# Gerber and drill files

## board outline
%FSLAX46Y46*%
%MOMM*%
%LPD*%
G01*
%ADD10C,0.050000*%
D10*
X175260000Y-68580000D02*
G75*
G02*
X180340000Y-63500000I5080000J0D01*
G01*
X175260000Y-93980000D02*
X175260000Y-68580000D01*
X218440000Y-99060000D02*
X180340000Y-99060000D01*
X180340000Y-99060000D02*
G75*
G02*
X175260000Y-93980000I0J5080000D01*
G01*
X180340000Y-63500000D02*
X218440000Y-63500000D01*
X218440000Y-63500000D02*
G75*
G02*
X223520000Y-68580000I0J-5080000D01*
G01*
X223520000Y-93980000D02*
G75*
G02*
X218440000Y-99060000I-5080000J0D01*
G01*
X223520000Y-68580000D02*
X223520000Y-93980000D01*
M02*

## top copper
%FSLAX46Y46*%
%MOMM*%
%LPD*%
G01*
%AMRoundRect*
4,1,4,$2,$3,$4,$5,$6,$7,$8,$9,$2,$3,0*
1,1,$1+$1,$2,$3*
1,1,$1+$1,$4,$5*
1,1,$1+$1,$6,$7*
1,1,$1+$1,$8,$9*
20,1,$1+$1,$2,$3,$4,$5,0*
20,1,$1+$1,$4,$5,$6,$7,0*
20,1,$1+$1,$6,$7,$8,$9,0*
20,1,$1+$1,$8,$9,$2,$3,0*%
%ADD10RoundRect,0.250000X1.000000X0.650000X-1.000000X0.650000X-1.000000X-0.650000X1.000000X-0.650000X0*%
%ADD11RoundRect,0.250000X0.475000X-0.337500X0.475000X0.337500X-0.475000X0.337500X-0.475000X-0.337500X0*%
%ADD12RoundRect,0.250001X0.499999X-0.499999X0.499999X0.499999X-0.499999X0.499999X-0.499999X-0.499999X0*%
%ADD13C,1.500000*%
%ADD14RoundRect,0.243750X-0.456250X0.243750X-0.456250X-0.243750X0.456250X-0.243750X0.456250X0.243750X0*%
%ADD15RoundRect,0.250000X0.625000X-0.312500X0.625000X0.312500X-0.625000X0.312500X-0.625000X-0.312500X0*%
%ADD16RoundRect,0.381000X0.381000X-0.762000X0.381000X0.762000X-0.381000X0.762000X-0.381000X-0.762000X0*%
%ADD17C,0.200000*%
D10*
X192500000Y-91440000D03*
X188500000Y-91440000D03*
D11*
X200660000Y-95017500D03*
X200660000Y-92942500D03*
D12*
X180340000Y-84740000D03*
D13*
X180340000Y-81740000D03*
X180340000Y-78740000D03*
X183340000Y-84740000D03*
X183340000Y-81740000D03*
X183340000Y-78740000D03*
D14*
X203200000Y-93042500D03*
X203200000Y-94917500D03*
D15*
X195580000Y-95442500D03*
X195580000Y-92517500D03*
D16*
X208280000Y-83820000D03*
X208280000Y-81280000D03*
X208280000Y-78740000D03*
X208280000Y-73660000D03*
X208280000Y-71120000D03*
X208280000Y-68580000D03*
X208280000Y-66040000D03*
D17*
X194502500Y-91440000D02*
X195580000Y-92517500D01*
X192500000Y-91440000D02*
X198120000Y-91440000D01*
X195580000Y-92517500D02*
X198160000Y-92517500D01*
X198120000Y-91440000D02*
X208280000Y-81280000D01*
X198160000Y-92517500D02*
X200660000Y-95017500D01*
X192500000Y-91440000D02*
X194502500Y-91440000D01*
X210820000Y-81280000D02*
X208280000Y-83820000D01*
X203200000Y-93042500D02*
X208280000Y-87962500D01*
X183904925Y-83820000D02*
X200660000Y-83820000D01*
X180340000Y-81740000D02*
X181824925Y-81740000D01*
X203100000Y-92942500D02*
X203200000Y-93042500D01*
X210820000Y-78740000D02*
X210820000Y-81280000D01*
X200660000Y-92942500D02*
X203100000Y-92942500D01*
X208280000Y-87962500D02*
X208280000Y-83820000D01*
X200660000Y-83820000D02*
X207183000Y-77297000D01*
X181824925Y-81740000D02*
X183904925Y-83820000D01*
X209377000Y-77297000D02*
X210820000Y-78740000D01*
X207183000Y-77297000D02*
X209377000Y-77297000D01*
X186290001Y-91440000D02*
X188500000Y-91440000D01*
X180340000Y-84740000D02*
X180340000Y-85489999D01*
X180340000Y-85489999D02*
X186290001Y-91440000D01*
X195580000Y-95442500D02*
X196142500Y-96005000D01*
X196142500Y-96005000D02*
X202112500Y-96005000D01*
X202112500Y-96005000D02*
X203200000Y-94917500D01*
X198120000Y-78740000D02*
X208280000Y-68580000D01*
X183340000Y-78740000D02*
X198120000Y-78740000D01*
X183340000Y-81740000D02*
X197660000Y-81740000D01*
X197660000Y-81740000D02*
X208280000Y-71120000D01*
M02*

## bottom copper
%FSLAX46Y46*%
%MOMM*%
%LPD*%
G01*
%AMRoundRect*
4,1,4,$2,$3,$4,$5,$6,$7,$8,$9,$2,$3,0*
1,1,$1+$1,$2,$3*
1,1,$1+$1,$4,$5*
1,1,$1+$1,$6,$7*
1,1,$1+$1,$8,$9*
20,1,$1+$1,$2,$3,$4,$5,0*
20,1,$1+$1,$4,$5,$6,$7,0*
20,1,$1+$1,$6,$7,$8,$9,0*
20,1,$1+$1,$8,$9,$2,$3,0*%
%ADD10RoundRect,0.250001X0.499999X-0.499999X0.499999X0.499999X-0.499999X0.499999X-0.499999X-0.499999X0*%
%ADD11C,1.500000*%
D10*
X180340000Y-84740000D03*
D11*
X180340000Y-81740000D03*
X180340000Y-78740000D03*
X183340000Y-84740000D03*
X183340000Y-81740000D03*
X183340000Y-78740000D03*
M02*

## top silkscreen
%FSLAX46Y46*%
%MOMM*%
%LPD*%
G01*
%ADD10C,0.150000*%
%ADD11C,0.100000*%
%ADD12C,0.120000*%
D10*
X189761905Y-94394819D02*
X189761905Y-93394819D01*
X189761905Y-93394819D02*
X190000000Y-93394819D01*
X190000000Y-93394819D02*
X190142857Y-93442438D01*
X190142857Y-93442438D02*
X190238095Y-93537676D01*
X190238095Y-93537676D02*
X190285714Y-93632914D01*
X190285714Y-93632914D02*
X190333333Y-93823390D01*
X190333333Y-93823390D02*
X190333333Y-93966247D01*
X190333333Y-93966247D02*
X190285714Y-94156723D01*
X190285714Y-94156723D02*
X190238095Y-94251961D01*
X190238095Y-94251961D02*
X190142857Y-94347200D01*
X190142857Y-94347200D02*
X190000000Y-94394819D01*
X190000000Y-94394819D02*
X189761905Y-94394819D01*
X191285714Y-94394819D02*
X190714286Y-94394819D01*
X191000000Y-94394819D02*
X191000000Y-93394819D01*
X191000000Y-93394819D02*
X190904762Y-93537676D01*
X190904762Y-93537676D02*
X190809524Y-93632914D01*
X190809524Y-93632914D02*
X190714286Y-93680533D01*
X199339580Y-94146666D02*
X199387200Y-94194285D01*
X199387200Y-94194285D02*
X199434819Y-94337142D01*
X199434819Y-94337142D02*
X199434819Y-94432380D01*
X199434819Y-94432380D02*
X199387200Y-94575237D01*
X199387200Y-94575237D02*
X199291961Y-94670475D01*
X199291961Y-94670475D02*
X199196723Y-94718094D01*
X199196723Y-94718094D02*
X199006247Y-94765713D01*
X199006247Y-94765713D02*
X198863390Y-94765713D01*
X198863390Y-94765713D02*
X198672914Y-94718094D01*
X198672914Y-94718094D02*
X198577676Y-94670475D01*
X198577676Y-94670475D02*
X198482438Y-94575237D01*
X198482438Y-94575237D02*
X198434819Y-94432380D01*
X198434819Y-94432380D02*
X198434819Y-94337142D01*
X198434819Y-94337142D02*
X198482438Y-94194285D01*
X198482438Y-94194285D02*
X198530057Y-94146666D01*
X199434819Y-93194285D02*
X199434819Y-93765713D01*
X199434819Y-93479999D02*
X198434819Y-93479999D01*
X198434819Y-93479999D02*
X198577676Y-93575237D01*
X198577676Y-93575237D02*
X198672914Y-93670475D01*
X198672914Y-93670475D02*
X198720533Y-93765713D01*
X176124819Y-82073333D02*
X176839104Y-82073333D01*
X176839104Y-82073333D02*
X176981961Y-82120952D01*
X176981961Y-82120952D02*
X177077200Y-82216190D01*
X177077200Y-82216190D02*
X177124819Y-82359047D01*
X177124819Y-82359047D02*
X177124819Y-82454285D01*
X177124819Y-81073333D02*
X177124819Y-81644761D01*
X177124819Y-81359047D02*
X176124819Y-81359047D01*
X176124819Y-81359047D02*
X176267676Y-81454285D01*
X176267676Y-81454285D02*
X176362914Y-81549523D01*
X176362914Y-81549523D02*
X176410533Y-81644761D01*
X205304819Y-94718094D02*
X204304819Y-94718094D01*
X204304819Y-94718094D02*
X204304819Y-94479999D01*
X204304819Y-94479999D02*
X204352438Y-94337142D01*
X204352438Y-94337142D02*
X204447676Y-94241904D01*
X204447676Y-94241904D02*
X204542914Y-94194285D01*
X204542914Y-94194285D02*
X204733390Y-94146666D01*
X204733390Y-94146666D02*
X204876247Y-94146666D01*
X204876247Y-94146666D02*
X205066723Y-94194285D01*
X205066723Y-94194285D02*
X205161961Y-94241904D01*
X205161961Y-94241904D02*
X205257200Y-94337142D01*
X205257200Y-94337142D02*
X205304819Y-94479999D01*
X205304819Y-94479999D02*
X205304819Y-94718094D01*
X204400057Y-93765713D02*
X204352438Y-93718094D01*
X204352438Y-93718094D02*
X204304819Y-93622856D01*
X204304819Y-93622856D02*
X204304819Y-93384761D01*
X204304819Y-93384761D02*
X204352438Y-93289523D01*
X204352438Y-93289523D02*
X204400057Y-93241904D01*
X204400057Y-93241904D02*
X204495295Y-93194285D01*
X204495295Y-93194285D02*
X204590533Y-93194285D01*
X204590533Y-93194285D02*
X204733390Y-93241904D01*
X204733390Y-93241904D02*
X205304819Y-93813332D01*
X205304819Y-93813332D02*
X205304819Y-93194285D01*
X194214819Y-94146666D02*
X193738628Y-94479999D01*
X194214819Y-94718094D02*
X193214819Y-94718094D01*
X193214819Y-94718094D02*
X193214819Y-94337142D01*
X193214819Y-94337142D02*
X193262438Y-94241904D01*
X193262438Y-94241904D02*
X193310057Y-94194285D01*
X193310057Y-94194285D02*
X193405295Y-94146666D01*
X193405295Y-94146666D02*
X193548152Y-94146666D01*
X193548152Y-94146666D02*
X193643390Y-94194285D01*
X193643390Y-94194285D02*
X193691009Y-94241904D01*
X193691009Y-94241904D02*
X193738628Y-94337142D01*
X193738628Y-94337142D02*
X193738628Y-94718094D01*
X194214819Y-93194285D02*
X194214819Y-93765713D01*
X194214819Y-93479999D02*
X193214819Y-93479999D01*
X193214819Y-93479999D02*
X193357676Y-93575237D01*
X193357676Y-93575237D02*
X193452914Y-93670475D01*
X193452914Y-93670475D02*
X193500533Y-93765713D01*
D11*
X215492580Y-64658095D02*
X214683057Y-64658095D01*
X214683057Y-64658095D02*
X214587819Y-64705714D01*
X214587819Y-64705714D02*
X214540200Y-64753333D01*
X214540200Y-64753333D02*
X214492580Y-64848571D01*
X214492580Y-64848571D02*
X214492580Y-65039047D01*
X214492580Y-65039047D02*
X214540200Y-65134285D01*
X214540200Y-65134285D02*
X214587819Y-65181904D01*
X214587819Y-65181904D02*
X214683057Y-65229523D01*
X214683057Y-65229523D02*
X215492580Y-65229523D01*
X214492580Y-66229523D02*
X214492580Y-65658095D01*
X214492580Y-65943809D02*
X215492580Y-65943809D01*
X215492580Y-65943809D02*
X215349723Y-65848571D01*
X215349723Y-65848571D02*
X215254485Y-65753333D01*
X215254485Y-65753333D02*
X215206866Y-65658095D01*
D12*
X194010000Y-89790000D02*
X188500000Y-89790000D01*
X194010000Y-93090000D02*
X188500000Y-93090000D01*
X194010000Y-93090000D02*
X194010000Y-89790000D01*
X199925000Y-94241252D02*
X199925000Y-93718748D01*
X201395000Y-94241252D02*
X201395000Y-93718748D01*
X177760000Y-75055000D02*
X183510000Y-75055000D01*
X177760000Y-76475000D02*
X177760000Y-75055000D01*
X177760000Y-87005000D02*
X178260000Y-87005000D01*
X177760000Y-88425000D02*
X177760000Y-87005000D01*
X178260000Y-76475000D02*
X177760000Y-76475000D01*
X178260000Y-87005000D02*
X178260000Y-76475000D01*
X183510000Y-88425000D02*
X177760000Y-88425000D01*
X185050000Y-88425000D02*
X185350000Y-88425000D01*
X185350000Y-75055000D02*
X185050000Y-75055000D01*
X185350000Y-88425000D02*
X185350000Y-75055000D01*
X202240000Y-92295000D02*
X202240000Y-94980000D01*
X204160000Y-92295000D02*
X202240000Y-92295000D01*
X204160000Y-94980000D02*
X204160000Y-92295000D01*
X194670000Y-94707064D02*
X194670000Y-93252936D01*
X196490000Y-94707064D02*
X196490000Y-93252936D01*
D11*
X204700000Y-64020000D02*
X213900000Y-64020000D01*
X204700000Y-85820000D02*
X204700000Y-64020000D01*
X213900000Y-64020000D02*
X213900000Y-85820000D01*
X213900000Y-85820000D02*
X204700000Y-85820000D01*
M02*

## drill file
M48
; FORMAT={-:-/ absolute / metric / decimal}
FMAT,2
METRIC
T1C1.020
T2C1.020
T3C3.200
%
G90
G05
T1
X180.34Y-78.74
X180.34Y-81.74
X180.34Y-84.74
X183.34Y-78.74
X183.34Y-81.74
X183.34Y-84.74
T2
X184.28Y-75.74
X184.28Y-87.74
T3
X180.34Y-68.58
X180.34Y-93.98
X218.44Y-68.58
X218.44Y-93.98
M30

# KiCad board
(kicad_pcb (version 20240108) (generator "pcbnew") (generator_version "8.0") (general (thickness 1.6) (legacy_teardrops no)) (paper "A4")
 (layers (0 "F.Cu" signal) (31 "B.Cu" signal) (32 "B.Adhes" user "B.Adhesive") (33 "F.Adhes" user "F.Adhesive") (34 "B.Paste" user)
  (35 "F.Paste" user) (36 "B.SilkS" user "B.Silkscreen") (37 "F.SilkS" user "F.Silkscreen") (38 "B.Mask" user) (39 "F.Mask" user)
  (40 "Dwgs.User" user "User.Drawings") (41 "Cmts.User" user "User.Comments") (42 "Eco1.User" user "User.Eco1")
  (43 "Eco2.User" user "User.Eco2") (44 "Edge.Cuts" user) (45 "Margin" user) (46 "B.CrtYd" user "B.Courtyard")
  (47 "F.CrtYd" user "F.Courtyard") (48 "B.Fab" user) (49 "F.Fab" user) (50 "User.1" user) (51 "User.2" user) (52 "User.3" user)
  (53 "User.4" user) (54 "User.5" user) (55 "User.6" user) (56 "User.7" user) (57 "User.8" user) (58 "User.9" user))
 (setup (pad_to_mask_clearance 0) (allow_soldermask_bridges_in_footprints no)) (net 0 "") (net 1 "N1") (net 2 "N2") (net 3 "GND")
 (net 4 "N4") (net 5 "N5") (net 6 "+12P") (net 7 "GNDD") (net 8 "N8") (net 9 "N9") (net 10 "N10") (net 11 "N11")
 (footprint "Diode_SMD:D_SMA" (layer "F.Cu") (at 190.5 91.44 180)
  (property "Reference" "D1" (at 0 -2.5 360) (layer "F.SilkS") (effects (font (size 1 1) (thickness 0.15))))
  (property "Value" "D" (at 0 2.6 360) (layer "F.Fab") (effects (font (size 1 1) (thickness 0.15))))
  (fp_line (start -3.51 1.65) (end 2 1.65) (stroke (width 0.12) (type solid)) (layer "F.SilkS"))
  (fp_line (start -3.51 -1.65) (end 2 -1.65) (stroke (width 0.12) (type solid)) (layer "F.SilkS"))
  (fp_line (start -3.51 -1.65) (end -3.51 1.65) (stroke (width 0.12) (type solid)) (layer "F.SilkS"))
  (pad "1" smd roundrect (at -2 0 180) (size 2.5 1.8) (layers "F.Cu" "F.Paste" "F.Mask") (roundrect_rratio 0.1388888889) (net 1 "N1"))
  (pad "2" smd roundrect (at 2 0 180) (size 2.5 1.8) (layers "F.Cu" "F.Paste" "F.Mask") (roundrect_rratio 0.1388888889) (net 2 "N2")))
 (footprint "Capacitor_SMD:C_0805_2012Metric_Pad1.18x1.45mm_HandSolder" (layer "F.Cu") (at 200.66 93.98 90)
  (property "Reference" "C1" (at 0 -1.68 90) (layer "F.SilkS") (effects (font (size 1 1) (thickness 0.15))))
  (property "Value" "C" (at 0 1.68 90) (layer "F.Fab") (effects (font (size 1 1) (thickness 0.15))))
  (fp_line (start -0.261252 -0.735) (end 0.261252 -0.735) (stroke (width 0.12) (type solid)) (layer "F.SilkS"))
  (fp_line (start -0.261252 0.735) (end 0.261252 0.735) (stroke (width 0.12) (type solid)) (layer "F.SilkS"))
  (pad "1" smd roundrect (at -1.0375 0 90) (size 1.175 1.45) (layers "F.Cu" "F.Paste" "F.Mask") (roundrect_rratio 0.212766) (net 1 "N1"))
  (pad "2" smd roundrect (at 1.0375 0 90) (size 1.175 1.45) (layers "F.Cu" "F.Paste" "F.Mask") (roundrect_rratio 0.212766) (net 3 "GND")))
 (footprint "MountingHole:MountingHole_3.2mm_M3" (layer "F.Cu") (at 218.44 93.98)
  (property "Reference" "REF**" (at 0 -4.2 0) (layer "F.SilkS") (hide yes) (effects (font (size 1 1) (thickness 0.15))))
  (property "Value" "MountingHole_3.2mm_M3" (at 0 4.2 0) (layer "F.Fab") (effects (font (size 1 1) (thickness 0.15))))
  (pad "" np_thru_hole circle (at 0 0) (size 3.2 3.2) (drill 3.2) (layers "*.Cu" "*.Mask")))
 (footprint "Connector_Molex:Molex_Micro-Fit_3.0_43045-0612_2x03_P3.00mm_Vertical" (layer "F.Cu") (at 180.34 84.74 90)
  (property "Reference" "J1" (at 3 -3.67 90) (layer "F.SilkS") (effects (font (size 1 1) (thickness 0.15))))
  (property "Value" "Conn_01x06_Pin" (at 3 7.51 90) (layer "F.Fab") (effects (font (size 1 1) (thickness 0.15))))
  (fp_line (start 9.685 -2.58) (end 9.685 3.17) (stroke (width 0.12) (type solid)) (layer "F.SilkS"))
  (fp_line (start 8.265 -2.58) (end 9.685 -2.58) (stroke (width 0.12) (type solid)) (layer "F.SilkS"))
  (fp_line (start -2.265 -2.58) (end -2.265 -2.08) (stroke (width 0.12) (type solid)) (layer "F.SilkS"))
  (fp_line (start -3.685 -2.58) (end -2.265 -2.58) (stroke (width 0.12) (type solid)) (layer "F.SilkS"))
  (fp_line (start 8.265 -2.08) (end 8.265 -2.58) (stroke (width 0.12) (type solid)) (layer "F.SilkS"))
  (fp_line (start -2.265 -2.08) (end 8.265 -2.08) (stroke (width 0.12) (type solid)) (layer "F.SilkS"))
  (fp_line (start -3.685 3.17) (end -3.685 -2.58) (stroke (width 0.12) (type solid)) (layer "F.SilkS"))
  (fp_line (start -3.685 4.71) (end -3.685 5.01) (stroke (width 0.12) (type solid)) (layer "F.SilkS"))
  (fp_line (start 9.685 5.01) (end 9.685 4.71) (stroke (width 0.12) (type solid)) (layer "F.SilkS"))
  (fp_line (start -3.685 5.01) (end 9.685 5.01) (stroke (width 0.12) (type solid)) (layer "F.SilkS"))
  (pad "" np_thru_hole circle (at -3 3.94 90) (size 1.02 1.02) (drill 1.02) (layers "*.Cu" "*.Mask"))
  (pad "" np_thru_hole circle (at 9 3.94 90) (size 1.02 1.02) (drill 1.02) (layers "*.Cu" "*.Mask"))
  (pad "1" thru_hole roundrect (at 0 0 90) (size 1.5 1.5) (drill 1.02) (layers "*.Cu" "*.Mask") (remove_unused_layers no)
   (roundrect_rratio 0.166667) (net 2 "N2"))
  (pad "2" thru_hole circle (at 3 0 90) (size 1.5 1.5) (drill 1.02) (layers "*.Cu" "*.Mask") (remove_unused_layers no) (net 3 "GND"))
  (pad "3" thru_hole circle (at 6 0 90) (size 1.5 1.5) (drill 1.02) (layers "*.Cu" "*.Mask") (remove_unused_layers no) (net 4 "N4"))
  (pad "4" thru_hole circle (at 0 3 90) (size 1.5 1.5) (drill 1.02) (layers "*.Cu" "*.Mask") (remove_unused_layers no) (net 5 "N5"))
  (pad "5" thru_hole circle (at 3 3 90) (size 1.5 1.5) (drill 1.02) (layers "*.Cu" "*.Mask") (remove_unused_layers no) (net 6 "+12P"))
  (pad "6" thru_hole circle (at 6 3 90) (size 1.5 1.5) (drill 1.02) (layers "*.Cu" "*.Mask") (remove_unused_layers no) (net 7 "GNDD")))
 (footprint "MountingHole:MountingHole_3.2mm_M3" (layer "F.Cu") (at 180.34 93.98)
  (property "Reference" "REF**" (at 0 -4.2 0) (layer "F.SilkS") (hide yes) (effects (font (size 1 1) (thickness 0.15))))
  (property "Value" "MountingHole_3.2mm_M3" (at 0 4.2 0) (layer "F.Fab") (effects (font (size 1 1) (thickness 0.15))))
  (pad "" np_thru_hole circle (at 0 0) (size 3.2 3.2) (drill 3.2) (layers "*.Cu" "*.Mask")))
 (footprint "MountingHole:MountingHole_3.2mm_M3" (layer "F.Cu") (at 180.34 68.58)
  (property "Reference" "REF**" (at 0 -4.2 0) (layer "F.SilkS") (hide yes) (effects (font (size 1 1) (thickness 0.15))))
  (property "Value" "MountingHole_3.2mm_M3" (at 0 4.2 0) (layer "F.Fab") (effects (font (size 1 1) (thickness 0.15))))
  (pad "" np_thru_hole circle (at 0 0) (size 3.2 3.2) (drill 3.2) (layers "*.Cu" "*.Mask")))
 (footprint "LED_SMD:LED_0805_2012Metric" (layer "F.Cu") (at 203.2 93.98 -90)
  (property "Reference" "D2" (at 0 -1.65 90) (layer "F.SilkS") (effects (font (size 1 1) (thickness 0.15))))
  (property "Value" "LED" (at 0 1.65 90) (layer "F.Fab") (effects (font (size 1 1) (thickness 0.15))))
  (fp_line (start -1.685 0.96) (end 1 0.96) (stroke (width 0.12) (type solid)) (layer "F.SilkS"))
  (fp_line (start -1.685 -0.96) (end -1.685 0.96) (stroke (width 0.12) (type solid)) (layer "F.SilkS"))
  (fp_line (start 1 -0.96) (end -1.685 -0.96) (stroke (width 0.12) (type solid)) (layer "F.SilkS"))
  (pad "1" smd roundrect (at -0.9375 0 270) (size 0.975 1.4) (layers "F.Cu" "F.Paste" "F.Mask") (roundrect_rratio 0.25) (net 3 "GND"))
  (pad "2" smd roundrect (at 0.9375 0 270) (size 0.975 1.4) (layers "F.Cu" "F.Paste" "F.Mask") (roundrect_rratio 0.25) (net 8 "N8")))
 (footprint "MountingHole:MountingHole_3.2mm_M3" (layer "F.Cu") (at 218.44 68.58)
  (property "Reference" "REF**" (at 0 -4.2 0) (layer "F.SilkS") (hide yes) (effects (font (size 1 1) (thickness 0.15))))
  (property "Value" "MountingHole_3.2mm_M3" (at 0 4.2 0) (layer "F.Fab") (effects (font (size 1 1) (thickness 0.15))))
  (pad "" np_thru_hole circle (at 0 0) (size 3.2 3.2) (drill 3.2) (layers "*.Cu" "*.Mask")))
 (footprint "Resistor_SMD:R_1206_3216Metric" (layer "F.Cu") (at 195.58 93.98 90)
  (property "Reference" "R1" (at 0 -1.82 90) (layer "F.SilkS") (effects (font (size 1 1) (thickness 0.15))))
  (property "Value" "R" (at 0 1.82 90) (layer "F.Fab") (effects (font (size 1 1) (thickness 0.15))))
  (fp_line (start -0.727064 -0.91) (end 0.727064 -0.91) (stroke (width 0.12) (type solid)) (layer "F.SilkS"))
  (fp_line (start -0.727064 0.91) (end 0.727064 0.91) (stroke (width 0.12) (type solid)) (layer "F.SilkS"))
  (pad "1" smd roundrect (at -1.4625 0 90) (size 1.125 1.75) (layers "F.Cu" "F.Paste" "F.Mask") (roundrect_rratio 0.222222) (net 8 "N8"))
  (pad "2" smd roundrect (at 1.4625 0 90) (size 1.125 1.75) (layers "F.Cu" "F.Paste" "F.Mask") (roundrect_rratio 0.222222) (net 1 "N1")))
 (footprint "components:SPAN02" (layer "F.Cu") (at 203.2 83.82 90)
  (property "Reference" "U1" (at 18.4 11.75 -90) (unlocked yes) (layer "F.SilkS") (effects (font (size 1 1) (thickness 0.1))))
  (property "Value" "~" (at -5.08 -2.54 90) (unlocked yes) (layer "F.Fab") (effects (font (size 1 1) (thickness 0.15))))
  (fp_line (start 19.8 1.5) (end 19.8 10.7) (stroke (width 0.1) (type default)) (layer "F.SilkS"))
  (fp_line (start -2 1.5) (end 19.8 1.5) (stroke (width 0.1) (type default)) (layer "F.SilkS"))
  (fp_line (start 19.8 10.7) (end -2 10.7) (stroke (width 0.1) (type default)) (layer "F.SilkS"))
  (fp_line (start -2 10.7) (end -2 1.5) (stroke (width 0.1) (type default)) (layer "F.SilkS"))
  (pad "1" smd roundrect (at 0 5.08 90) (size 2.286 1.524) (layers "F.Cu" "F.Paste" "F.Mask") (roundrect_rratio 0.25) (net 3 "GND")
   (thermal_bridge_angle 45))
  (pad "2" smd roundrect (at 2.54 5.08 90) (size 2.286 1.524) (layers "F.Cu" "F.Paste" "F.Mask") (roundrect_rratio 0.25) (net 1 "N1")
   (thermal_bridge_angle 45))
  (pad "3" smd roundrect (at 5.08 5.08 90) (size 2.286 1.524) (layers "F.Cu" "F.Paste" "F.Mask") (roundrect_rratio 0.25) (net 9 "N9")
   (thermal_bridge_angle 45))
  (pad "5" smd roundrect (at 10.16 5.08 90) (size 2.286 1.524) (layers "F.Cu" "F.Paste" "F.Mask") (roundrect_rratio 0.25) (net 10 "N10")
   (thermal_bridge_angle 45))
  (pad "6" smd roundrect (at 12.7 5.08 90) (size 2.286 1.524) (layers "F.Cu" "F.Paste" "F.Mask") (roundrect_rratio 0.25) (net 6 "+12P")
   (thermal_bridge_angle 45))
  (pad "7" smd roundrect (at 15.24 5.08 90) (size 2.286 1.524) (layers "F.Cu" "F.Paste" "F.Mask") (roundrect_rratio 0.25) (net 7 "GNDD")
   (thermal_bridge_angle 45))
  (pad "8" smd roundrect (at 17.78 5.08 90) (size 2.286 1.524) (layers "F.Cu" "F.Paste" "F.Mask") (roundrect_rratio 0.25) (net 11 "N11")
   (thermal_bridge_angle 45)))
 (gr_arc (start 175.26 68.58) (mid 176.747898 64.987898) (end 180.34 63.5) (stroke (width 0.05) (type default)) (layer "Edge.Cuts"))
 (gr_line (start 175.26 93.98) (end 175.26 68.58) (stroke (width 0.05) (type default)) (layer "Edge.Cuts"))
 (gr_line (start 218.44 99.06) (end 180.34 99.06) (stroke (width 0.05) (type default)) (layer "Edge.Cuts"))
 (gr_arc (start 180.34 99.06) (mid 176.747898 97.572102) (end 175.26 93.98) (stroke (width 0.05) (type default)) (layer "Edge.Cuts"))
 (gr_line (start 180.34 63.5) (end 218.44 63.5) (stroke (width 0.05) (type default)) (layer "Edge.Cuts"))
 (gr_arc (start 218.44 63.5) (mid 222.032102 64.987898) (end 223.52 68.58) (stroke (width 0.05) (type default)) (layer "Edge.Cuts"))
 (gr_arc (start 223.52 93.98) (mid 222.032102 97.572102) (end 218.44 99.06) (stroke (width 0.05) (type default)) (layer "Edge.Cuts"))
 (gr_line (start 223.52 68.58) (end 223.52 93.98) (stroke (width 0.05) (type default)) (layer "Edge.Cuts"))
 (segment (start 194.5025 91.44) (end 195.58 92.5175) (width 0.2) (layer "F.Cu") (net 1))
 (segment (start 192.5 91.44) (end 198.12 91.44) (width 0.2) (layer "F.Cu") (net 1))
 (segment (start 195.58 92.5175) (end 198.16 92.5175) (width 0.2) (layer "F.Cu") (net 1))
 (segment (start 198.12 91.44) (end 208.28 81.28) (width 0.2) (layer "F.Cu") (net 1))
 (segment (start 198.16 92.5175) (end 200.66 95.0175) (width 0.2) (layer "F.Cu") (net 1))
 (segment (start 192.5 91.44) (end 194.5025 91.44) (width 0.2) (layer "F.Cu") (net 1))
 (segment (start 210.82 81.28) (end 208.28 83.82) (width 0.2) (layer "F.Cu") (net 3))
 (segment (start 203.2 93.0425) (end 208.28 87.9625) (width 0.2) (layer "F.Cu") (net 3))
 (segment (start 183.904925 83.82) (end 200.66 83.82) (width 0.2) (layer "F.Cu") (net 3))
 (segment (start 180.34 81.74) (end 181.824925 81.74) (width 0.2) (layer "F.Cu") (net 3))
 (segment (start 203.1 92.9425) (end 203.2 93.0425) (width 0.2) (layer "F.Cu") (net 3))
 (segment (start 210.82 78.74) (end 210.82 81.28) (width 0.2) (layer "F.Cu") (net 3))
 (segment (start 200.66 92.9425) (end 203.1 92.9425) (width 0.2) (layer "F.Cu") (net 3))
 (segment (start 208.28 87.9625) (end 208.28 83.82) (width 0.2) (layer "F.Cu") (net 3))
 (segment (start 200.66 83.82) (end 207.183 77.297) (width 0.2) (layer "F.Cu") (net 3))
 (segment (start 181.824925 81.74) (end 183.904925 83.82) (width 0.2) (layer "F.Cu") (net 3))
 (segment (start 209.377 77.297) (end 210.82 78.74) (width 0.2) (layer "F.Cu") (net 3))
 (segment (start 207.183 77.297) (end 209.377 77.297) (width 0.2) (layer "F.Cu") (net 3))
 (segment (start 186.290001 91.44) (end 188.5 91.44) (width 0.2) (layer "F.Cu") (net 2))
 (segment (start 180.34 84.74) (end 180.34 85.489999) (width 0.2) (layer "F.Cu") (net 2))
 (segment (start 180.34 85.489999) (end 186.290001 91.44) (width 0.2) (layer "F.Cu") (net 2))
 (segment (start 195.58 95.4425) (end 196.1425 96.005) (width 0.2) (layer "F.Cu") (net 8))
 (segment (start 196.1425 96.005) (end 202.1125 96.005) (width 0.2) (layer "F.Cu") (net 8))
 (segment (start 202.1125 96.005) (end 203.2 94.9175) (width 0.2) (layer "F.Cu") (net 8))
 (segment (start 198.12 78.74) (end 208.28 68.58) (width 0.2) (layer "F.Cu") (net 7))
 (segment (start 183.34 78.74) (end 198.12 78.74) (width 0.2) (layer "F.Cu") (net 7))
 (segment (start 183.34 81.74) (end 197.66 81.74) (width 0.2) (layer "F.Cu") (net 6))
 (segment (start 197.66 81.74) (end 208.28 71.12) (width 0.2) (layer "F.Cu") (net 6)))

